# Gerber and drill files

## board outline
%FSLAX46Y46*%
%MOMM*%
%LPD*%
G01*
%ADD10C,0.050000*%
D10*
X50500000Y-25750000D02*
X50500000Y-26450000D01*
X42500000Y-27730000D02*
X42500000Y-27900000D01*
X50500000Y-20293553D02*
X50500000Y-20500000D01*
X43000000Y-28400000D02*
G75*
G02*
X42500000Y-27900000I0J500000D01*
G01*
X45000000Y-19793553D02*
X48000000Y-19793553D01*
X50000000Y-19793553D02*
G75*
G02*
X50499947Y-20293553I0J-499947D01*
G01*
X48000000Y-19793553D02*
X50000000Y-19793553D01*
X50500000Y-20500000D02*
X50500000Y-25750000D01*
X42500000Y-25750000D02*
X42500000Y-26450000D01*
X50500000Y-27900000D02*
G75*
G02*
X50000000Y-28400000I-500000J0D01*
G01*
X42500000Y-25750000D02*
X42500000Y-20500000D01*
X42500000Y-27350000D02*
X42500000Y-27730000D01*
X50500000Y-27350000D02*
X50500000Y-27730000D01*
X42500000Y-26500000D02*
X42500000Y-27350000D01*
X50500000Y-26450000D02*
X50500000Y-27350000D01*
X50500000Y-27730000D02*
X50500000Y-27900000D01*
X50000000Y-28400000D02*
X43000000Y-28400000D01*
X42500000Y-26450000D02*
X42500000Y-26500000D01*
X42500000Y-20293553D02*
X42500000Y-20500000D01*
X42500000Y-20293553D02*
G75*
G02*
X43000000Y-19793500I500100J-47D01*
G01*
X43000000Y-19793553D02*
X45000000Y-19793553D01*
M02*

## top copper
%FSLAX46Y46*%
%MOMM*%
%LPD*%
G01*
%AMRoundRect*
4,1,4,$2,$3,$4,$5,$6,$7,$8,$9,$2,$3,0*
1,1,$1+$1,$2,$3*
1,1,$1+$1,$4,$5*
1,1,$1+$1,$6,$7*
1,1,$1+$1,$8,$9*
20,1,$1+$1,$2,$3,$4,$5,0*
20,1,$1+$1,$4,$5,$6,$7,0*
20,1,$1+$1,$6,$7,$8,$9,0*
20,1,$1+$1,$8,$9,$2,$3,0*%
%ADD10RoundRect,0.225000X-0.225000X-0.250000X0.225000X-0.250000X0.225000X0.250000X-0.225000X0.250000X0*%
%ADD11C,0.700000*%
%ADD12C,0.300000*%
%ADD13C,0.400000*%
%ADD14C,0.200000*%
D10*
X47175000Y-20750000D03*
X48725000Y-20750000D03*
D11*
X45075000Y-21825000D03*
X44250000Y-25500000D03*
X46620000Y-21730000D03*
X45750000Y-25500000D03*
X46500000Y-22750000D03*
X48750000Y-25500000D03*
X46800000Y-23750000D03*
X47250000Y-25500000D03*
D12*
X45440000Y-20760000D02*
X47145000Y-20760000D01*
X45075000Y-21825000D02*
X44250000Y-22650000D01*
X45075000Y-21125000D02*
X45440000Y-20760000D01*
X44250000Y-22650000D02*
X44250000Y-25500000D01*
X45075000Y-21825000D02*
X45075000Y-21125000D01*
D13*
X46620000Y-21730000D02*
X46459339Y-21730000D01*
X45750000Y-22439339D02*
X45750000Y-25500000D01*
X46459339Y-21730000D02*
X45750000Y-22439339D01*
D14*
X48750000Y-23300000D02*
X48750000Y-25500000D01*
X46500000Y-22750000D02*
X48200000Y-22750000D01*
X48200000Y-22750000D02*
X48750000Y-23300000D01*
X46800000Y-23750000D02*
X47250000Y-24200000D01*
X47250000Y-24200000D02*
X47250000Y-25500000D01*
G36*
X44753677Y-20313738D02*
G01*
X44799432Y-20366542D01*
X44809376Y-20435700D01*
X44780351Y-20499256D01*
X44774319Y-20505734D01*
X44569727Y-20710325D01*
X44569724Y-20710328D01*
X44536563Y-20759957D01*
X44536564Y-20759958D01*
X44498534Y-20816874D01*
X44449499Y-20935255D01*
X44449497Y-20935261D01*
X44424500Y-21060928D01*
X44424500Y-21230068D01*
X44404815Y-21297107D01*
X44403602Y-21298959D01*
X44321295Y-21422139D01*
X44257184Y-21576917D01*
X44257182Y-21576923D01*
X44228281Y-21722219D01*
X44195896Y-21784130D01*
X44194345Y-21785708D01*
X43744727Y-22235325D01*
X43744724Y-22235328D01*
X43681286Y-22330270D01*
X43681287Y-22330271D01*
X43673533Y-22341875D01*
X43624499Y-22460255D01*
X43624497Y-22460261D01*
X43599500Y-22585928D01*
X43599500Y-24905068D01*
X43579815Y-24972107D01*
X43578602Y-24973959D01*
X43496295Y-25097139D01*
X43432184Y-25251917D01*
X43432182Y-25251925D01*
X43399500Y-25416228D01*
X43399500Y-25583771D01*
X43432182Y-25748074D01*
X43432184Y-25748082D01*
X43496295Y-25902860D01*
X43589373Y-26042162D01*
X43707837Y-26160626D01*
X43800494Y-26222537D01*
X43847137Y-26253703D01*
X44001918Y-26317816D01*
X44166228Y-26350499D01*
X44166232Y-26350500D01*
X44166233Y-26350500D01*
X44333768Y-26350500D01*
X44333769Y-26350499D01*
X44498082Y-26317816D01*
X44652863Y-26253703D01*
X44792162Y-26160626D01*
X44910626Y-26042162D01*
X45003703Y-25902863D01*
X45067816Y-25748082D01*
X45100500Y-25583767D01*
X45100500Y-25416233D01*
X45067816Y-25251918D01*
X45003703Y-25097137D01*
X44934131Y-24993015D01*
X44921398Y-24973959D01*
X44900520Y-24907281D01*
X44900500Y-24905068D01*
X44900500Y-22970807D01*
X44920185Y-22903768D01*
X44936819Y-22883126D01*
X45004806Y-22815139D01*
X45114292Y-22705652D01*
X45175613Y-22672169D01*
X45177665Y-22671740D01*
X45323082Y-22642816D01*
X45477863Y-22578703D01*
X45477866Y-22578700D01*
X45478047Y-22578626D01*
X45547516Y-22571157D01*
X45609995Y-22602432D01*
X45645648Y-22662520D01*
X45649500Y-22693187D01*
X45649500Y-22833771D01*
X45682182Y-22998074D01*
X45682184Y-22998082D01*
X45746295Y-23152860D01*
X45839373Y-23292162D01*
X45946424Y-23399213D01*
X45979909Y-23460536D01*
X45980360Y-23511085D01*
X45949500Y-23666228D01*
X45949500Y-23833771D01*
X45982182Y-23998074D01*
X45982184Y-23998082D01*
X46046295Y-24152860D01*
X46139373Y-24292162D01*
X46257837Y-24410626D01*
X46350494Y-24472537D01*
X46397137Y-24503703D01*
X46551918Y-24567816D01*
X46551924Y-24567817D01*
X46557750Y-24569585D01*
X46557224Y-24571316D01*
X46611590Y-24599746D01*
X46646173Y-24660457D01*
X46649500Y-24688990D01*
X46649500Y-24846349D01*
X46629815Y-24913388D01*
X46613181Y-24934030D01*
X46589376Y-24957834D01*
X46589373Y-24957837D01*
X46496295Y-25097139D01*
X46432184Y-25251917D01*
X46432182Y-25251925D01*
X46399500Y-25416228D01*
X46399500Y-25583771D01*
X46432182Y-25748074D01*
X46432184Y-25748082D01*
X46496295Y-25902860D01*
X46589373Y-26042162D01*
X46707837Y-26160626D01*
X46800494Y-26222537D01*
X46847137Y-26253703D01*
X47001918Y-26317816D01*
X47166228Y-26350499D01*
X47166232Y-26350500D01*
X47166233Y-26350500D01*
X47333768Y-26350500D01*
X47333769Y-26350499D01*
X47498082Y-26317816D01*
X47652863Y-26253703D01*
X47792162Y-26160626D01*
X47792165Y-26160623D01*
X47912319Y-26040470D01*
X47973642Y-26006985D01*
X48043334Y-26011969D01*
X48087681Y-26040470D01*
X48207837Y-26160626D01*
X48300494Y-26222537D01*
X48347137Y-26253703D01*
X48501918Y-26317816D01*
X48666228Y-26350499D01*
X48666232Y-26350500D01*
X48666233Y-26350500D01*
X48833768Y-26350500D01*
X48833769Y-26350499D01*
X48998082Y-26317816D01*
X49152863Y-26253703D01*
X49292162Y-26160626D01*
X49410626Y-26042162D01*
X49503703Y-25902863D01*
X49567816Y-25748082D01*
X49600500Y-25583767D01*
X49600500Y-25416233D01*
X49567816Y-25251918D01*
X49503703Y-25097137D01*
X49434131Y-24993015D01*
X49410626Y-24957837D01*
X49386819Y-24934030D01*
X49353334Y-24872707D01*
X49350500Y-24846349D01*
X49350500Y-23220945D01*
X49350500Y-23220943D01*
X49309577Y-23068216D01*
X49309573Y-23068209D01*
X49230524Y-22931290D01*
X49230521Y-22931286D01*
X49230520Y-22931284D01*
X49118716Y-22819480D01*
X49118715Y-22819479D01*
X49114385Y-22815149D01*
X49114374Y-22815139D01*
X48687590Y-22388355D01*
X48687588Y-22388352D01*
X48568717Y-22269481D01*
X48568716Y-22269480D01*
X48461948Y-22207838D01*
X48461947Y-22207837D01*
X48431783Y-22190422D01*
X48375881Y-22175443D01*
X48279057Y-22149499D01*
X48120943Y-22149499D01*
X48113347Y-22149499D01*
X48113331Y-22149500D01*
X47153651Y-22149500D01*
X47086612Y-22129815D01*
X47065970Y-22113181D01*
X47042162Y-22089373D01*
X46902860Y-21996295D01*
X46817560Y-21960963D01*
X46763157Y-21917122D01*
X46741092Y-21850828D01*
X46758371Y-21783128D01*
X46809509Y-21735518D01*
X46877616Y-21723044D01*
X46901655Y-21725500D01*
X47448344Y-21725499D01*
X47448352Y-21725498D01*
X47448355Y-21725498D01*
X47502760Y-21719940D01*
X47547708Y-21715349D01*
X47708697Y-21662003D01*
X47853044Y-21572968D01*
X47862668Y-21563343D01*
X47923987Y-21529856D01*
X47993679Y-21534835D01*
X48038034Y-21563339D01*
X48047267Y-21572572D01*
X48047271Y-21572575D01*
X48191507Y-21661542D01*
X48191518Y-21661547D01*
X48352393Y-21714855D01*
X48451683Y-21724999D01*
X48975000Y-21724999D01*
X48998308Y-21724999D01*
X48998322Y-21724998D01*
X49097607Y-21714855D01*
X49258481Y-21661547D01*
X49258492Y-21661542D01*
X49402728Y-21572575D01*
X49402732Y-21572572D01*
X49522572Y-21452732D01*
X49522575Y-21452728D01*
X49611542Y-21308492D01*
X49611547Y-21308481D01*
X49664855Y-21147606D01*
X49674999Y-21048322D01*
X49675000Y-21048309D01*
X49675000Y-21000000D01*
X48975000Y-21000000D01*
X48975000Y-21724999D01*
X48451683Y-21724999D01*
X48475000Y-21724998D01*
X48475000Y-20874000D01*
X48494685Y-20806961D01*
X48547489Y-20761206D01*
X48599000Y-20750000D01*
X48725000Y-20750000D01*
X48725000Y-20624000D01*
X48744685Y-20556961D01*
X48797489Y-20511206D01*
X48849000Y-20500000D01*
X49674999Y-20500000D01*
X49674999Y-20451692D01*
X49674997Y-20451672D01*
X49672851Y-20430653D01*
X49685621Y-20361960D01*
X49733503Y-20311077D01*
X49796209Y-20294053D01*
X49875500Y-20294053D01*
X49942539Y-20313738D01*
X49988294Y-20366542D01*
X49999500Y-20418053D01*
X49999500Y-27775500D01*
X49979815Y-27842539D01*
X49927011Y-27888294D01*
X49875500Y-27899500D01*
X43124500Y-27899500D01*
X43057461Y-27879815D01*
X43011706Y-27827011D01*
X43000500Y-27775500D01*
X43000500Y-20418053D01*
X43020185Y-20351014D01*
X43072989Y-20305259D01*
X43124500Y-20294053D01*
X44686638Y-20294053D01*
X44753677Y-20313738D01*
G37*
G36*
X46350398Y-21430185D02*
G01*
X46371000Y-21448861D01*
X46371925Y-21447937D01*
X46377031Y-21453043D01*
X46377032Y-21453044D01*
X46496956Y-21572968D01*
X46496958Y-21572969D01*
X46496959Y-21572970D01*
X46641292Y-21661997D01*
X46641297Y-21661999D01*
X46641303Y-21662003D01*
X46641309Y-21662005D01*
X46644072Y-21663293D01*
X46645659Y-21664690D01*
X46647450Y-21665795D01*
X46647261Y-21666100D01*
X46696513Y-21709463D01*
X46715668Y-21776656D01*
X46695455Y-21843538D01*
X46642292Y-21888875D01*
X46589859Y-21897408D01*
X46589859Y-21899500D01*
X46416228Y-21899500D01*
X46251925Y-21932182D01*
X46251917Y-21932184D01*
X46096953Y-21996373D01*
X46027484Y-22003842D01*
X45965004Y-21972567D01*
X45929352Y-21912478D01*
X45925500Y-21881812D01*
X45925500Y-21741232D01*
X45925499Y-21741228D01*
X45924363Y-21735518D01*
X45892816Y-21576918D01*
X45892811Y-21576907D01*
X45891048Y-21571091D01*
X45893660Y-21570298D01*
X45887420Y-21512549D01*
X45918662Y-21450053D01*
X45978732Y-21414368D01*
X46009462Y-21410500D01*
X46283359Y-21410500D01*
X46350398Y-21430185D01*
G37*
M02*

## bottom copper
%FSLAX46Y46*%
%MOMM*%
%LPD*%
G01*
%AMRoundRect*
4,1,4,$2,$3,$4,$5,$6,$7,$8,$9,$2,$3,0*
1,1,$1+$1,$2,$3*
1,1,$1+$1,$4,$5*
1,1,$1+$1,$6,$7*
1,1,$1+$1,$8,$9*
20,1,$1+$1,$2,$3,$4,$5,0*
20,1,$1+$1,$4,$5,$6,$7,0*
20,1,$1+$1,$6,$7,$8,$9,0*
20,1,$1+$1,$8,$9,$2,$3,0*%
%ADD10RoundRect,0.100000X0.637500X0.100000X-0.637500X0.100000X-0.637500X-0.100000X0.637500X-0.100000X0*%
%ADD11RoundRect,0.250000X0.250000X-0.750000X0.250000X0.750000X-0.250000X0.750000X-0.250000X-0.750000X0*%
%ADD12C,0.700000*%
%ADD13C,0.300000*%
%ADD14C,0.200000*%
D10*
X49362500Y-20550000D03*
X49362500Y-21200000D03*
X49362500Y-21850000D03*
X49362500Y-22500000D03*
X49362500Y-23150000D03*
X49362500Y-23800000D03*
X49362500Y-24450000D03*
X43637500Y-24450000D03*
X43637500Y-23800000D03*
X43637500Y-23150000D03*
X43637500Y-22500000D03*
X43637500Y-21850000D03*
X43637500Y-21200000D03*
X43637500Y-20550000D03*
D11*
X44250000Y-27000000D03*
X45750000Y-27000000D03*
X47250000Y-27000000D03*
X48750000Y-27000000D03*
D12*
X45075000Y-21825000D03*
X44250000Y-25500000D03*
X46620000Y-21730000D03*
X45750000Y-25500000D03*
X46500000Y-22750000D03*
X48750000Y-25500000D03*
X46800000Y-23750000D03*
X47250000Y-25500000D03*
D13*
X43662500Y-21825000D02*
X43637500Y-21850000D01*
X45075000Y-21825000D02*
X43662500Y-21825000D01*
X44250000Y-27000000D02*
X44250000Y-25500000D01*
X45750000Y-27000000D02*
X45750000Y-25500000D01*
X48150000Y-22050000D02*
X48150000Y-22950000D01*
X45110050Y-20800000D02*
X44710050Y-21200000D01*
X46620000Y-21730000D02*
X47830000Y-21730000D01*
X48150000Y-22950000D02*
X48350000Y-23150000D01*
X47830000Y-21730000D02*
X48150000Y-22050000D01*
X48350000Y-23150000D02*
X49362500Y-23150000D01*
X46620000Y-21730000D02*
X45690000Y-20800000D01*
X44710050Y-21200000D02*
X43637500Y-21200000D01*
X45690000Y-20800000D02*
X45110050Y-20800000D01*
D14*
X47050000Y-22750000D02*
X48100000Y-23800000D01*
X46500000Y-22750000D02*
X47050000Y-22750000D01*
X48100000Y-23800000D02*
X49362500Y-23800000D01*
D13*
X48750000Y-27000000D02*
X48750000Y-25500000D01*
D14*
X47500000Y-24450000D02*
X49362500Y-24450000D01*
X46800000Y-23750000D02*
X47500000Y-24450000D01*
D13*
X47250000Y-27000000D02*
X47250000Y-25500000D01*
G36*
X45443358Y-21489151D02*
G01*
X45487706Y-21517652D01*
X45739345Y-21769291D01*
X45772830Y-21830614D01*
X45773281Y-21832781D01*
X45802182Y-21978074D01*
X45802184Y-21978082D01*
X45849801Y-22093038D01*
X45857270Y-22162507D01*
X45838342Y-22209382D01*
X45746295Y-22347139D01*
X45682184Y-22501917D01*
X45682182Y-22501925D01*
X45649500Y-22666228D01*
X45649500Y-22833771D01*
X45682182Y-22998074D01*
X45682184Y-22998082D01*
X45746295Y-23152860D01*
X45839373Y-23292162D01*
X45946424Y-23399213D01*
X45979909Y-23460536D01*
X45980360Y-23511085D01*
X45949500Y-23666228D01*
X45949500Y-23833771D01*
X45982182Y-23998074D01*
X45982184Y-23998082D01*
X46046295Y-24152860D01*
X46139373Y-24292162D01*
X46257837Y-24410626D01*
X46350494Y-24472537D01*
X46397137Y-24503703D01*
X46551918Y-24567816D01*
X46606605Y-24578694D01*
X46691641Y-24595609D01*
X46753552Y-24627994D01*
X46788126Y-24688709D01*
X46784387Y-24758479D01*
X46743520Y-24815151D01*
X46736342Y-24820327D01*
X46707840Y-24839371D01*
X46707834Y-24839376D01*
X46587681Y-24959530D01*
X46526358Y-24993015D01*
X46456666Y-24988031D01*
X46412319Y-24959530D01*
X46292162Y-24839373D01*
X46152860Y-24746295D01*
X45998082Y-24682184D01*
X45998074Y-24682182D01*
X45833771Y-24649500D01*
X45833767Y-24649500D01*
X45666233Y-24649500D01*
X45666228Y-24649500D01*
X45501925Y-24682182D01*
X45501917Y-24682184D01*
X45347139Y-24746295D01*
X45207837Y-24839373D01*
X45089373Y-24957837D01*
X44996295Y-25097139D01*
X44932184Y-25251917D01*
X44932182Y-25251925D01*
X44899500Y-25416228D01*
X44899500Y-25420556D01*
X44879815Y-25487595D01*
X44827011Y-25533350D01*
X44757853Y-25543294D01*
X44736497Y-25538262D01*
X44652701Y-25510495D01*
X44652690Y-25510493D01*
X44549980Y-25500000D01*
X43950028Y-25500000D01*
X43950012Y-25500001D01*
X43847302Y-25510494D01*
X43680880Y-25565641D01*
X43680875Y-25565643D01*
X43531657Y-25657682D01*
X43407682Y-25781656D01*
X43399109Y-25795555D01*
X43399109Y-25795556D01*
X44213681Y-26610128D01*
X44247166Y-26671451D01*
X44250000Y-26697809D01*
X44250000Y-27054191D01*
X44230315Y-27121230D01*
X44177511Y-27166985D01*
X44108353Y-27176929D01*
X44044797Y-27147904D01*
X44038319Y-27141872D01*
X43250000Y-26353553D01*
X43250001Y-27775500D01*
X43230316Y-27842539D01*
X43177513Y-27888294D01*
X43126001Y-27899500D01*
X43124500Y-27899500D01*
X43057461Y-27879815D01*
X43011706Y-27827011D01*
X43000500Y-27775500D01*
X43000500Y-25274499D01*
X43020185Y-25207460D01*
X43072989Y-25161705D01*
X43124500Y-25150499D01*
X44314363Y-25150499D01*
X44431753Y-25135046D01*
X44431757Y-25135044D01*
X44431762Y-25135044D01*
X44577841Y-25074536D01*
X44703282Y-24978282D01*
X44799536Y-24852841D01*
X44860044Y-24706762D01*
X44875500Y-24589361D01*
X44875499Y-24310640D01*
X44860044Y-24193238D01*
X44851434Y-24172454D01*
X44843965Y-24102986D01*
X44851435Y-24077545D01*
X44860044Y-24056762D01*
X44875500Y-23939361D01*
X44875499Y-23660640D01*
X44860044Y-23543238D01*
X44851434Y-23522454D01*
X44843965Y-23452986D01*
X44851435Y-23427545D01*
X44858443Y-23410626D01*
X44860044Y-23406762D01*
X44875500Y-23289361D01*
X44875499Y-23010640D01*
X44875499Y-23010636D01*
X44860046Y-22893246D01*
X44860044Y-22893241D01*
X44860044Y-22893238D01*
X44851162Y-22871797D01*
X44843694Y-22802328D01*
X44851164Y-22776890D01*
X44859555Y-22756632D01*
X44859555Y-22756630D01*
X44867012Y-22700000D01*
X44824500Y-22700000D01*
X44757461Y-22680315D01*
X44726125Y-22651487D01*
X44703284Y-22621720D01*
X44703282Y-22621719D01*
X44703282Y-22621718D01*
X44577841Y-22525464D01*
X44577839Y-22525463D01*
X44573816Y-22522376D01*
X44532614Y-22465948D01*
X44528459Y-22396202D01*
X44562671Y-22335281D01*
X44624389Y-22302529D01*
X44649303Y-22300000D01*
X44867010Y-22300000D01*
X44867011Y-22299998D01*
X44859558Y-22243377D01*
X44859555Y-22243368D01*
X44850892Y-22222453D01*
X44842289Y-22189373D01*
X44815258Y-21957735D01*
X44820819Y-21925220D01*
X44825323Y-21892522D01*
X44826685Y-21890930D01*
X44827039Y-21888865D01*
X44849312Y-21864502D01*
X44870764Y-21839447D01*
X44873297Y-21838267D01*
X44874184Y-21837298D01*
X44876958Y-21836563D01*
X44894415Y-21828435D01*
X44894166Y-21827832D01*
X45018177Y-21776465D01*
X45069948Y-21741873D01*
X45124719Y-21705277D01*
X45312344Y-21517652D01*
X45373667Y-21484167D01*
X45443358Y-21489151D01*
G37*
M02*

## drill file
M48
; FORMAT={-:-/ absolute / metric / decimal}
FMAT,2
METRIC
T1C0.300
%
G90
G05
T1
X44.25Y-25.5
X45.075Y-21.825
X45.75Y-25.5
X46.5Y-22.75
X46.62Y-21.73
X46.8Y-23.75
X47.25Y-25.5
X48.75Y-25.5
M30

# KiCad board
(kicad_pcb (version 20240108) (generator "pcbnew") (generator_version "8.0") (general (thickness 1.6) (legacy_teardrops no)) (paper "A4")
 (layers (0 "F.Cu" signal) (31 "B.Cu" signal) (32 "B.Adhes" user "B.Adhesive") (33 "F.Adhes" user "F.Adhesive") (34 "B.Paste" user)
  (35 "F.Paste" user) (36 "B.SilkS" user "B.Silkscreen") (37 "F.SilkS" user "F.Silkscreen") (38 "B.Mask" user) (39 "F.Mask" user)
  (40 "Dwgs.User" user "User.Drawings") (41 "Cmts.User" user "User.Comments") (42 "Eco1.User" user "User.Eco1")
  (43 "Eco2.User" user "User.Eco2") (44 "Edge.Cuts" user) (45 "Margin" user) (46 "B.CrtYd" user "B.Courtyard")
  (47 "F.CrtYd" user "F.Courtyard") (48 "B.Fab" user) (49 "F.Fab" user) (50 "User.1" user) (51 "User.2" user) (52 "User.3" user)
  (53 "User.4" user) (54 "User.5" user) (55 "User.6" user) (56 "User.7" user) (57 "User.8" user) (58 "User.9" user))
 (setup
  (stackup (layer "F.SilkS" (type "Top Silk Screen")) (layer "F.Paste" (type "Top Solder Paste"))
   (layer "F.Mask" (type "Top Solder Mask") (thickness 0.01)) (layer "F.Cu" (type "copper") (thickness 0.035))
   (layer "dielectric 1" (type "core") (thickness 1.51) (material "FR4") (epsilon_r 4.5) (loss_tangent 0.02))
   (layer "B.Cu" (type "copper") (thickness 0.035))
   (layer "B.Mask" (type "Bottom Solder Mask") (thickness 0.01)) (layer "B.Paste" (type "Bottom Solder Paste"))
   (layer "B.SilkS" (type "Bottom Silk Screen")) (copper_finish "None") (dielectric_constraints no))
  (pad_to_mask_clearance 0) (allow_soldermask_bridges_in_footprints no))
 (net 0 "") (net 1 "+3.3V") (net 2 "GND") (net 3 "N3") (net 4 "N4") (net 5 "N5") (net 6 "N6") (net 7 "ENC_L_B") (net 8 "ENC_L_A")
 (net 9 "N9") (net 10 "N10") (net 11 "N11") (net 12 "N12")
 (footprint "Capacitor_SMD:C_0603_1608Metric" (layer "F.Cu") (at 47.95 20.75)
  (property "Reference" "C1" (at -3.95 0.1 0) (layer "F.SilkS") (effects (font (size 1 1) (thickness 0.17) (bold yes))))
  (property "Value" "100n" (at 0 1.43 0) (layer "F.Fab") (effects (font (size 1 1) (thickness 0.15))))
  (pad "1" smd roundrect (at -0.775 0) (size 0.9 0.95) (layers "F.Cu" "F.Paste" "F.Mask") (roundrect_rratio 0.25) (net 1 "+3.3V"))
  (pad "2" smd roundrect (at 0.775 0) (size 0.9 0.95) (layers "F.Cu" "F.Paste" "F.Mask") (roundrect_rratio 0.25) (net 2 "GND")))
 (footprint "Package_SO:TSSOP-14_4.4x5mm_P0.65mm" (layer "B.Cu") (at 46.5 22.5 180)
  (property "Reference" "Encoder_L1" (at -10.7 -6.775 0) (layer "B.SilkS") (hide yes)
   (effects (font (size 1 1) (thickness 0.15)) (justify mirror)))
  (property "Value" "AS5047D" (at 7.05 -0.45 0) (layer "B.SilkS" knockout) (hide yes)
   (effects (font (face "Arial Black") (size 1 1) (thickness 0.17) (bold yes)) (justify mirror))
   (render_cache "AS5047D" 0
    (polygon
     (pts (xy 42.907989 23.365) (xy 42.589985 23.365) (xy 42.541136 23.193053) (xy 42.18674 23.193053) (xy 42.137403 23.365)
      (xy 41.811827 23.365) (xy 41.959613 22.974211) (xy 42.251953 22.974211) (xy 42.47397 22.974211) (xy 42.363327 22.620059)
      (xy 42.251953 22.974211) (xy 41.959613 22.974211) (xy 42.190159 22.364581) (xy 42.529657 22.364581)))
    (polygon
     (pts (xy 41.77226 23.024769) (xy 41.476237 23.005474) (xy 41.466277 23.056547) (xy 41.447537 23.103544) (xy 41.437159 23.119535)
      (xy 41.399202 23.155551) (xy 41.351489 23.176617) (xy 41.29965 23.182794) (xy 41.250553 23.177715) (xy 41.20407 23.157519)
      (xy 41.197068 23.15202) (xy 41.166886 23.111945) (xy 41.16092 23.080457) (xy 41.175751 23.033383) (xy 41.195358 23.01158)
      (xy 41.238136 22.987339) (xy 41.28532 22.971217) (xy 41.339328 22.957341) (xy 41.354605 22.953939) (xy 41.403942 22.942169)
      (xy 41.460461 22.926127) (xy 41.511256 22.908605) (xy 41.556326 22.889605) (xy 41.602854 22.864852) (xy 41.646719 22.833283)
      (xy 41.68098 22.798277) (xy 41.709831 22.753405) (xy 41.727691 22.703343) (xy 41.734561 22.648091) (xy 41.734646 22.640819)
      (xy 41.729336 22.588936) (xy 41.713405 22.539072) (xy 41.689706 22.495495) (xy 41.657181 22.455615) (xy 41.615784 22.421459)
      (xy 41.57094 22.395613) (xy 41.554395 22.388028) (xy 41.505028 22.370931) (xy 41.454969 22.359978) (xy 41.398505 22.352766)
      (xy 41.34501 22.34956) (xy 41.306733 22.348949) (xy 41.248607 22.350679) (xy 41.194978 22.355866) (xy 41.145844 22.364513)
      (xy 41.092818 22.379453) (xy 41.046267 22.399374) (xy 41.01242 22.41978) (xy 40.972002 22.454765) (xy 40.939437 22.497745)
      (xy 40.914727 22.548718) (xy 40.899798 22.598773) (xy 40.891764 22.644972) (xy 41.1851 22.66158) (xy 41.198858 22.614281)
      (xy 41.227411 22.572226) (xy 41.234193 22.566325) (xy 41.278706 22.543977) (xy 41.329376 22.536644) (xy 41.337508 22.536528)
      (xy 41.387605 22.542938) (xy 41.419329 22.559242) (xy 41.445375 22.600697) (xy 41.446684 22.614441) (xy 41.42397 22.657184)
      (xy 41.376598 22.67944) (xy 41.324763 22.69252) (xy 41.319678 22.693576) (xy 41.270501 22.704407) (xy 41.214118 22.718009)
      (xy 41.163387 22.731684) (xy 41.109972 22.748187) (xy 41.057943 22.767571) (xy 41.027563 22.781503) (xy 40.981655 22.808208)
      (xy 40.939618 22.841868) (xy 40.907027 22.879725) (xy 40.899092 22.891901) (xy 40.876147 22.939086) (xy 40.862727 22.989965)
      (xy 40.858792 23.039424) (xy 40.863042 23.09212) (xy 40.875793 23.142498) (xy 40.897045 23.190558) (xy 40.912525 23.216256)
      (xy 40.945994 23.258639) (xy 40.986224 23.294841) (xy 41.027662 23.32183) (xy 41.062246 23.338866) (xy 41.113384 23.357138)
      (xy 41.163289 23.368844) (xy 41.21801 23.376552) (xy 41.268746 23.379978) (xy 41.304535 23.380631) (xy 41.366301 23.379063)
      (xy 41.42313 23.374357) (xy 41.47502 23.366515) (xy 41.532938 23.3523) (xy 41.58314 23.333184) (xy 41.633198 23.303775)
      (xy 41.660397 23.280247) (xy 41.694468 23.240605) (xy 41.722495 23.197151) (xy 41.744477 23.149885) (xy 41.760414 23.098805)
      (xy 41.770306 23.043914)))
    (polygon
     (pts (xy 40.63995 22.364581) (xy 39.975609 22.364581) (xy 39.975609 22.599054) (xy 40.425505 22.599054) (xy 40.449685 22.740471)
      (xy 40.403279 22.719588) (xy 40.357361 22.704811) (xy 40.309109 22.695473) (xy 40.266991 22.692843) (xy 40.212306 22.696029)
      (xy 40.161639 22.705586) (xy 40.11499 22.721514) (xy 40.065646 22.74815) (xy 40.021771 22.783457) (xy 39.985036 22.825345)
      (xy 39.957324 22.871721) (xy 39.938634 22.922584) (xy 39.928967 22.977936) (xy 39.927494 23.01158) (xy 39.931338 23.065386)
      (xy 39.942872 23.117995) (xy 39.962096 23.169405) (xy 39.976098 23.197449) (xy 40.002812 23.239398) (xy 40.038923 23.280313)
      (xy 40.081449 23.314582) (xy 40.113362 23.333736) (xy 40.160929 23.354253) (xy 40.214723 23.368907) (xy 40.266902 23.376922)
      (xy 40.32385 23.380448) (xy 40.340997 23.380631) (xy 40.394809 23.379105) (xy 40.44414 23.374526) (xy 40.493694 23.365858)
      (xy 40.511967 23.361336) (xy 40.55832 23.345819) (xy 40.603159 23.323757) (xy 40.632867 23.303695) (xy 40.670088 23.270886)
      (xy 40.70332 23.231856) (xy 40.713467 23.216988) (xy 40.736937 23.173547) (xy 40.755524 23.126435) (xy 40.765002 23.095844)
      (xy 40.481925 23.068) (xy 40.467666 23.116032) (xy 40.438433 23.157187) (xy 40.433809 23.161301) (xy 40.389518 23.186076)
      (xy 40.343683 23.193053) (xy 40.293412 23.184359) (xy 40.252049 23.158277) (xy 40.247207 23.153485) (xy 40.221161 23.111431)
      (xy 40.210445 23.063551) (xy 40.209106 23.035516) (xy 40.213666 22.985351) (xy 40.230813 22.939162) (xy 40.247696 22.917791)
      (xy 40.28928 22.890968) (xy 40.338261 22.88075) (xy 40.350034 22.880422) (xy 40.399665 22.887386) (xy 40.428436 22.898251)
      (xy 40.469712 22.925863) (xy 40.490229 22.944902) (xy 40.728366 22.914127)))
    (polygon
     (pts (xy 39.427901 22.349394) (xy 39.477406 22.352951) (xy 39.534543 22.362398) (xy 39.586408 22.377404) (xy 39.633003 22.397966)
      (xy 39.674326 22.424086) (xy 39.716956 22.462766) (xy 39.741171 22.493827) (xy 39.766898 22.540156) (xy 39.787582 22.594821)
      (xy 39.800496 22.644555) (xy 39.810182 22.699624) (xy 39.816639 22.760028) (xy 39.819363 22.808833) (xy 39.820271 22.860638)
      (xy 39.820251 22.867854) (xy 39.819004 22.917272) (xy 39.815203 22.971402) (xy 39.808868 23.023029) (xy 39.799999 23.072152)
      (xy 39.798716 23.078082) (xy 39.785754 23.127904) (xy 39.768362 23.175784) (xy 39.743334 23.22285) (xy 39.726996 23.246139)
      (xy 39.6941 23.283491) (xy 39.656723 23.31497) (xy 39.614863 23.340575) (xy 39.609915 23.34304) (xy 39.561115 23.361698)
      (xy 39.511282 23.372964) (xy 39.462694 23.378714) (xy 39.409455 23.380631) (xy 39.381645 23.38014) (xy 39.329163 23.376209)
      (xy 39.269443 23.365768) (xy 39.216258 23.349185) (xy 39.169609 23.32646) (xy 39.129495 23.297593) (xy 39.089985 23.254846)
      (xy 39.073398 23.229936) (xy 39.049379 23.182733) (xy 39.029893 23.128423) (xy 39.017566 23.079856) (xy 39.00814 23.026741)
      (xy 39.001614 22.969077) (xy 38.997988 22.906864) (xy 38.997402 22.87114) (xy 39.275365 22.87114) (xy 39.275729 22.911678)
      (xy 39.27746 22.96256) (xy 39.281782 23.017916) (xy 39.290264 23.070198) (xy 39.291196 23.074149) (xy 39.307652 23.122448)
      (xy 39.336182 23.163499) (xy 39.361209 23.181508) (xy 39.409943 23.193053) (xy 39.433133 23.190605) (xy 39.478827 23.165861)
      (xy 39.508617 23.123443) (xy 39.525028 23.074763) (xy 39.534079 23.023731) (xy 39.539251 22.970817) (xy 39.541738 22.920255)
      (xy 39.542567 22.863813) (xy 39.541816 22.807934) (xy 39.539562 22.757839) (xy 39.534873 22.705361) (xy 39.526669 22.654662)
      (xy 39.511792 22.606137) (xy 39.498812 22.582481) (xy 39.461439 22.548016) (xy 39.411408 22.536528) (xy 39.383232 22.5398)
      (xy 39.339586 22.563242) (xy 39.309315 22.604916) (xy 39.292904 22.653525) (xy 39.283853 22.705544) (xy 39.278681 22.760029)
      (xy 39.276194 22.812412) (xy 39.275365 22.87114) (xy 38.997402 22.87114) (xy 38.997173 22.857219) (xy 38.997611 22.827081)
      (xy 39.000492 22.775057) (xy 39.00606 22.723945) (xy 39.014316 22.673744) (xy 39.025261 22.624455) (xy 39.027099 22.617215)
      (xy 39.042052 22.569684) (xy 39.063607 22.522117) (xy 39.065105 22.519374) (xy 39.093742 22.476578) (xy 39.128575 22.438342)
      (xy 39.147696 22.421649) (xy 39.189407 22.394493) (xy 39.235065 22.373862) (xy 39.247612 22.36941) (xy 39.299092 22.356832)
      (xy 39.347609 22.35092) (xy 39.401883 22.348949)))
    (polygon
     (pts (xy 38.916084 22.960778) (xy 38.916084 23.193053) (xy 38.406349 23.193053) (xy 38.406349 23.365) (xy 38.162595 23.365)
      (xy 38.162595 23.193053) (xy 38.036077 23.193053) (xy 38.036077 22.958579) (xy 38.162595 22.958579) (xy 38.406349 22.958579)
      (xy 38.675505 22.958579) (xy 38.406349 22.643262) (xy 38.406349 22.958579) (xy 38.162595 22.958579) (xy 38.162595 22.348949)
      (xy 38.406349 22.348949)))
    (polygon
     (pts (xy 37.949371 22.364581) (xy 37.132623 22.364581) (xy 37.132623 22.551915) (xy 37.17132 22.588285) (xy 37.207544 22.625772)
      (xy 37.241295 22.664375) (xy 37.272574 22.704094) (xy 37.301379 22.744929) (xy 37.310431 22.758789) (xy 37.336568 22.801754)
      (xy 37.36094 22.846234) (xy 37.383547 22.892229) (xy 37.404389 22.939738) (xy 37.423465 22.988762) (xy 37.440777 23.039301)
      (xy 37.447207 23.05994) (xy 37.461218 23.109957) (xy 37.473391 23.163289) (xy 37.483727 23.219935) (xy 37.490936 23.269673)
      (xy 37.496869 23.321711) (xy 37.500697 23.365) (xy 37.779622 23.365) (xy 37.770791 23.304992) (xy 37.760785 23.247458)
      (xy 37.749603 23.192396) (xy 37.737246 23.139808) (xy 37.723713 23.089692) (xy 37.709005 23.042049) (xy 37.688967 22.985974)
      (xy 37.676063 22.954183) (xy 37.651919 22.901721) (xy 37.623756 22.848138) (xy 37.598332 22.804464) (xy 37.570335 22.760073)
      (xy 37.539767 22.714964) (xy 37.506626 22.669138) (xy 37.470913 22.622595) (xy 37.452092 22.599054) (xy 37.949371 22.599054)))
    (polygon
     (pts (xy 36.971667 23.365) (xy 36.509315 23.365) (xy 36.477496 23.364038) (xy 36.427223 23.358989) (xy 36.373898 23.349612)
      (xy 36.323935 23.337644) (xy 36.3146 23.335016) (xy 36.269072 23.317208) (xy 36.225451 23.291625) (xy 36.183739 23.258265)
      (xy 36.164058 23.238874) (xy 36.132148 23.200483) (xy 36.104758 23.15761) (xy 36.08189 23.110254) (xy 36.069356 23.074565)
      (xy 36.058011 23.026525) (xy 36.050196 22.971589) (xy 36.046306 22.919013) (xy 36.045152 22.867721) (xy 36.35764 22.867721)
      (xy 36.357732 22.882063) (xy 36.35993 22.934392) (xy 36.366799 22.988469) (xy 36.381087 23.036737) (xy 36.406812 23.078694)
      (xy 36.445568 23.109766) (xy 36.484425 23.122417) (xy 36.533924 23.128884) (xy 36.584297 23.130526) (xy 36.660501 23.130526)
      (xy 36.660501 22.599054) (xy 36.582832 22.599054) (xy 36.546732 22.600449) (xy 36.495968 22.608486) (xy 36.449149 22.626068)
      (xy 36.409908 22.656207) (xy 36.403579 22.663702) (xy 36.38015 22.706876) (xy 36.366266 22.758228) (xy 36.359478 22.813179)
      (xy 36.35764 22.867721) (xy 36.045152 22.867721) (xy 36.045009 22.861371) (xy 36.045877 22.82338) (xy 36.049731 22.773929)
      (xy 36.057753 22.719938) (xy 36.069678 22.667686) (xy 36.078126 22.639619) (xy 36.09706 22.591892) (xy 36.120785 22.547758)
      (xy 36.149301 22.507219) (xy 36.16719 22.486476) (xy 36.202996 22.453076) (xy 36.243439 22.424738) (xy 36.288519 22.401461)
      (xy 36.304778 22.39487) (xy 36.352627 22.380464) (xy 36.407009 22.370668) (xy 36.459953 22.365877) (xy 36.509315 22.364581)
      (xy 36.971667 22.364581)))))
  (pad "1" smd roundrect (at -2.8625 1.95 180) (size 1.475 0.4) (layers "B.Cu" "B.Paste" "B.Mask") (roundrect_rratio 0.25) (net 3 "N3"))
  (pad "2" smd roundrect (at -2.8625 1.3 180) (size 1.475 0.4) (layers "B.Cu" "B.Paste" "B.Mask") (roundrect_rratio 0.25) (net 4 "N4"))
  (pad "3" smd roundrect (at -2.8625 0.65 180) (size 1.475 0.4) (layers "B.Cu" "B.Paste" "B.Mask") (roundrect_rratio 0.25) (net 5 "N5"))
  (pad "4" smd roundrect (at -2.8625 0 180) (size 1.475 0.4) (layers "B.Cu" "B.Paste" "B.Mask") (roundrect_rratio 0.25) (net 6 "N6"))
  (pad "5" smd roundrect (at -2.8625 -0.65 180) (size 1.475 0.4) (layers "B.Cu" "B.Paste" "B.Mask") (roundrect_rratio 0.25) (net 2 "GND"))
  (pad "6" smd roundrect (at -2.8625 -1.3 180) (size 1.475 0.4) (layers "B.Cu" "B.Paste" "B.Mask") (roundrect_rratio 0.25) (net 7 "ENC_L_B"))
  (pad "7" smd roundrect (at -2.8625 -1.95 180) (size 1.475 0.4) (layers "B.Cu" "B.Paste" "B.Mask") (roundrect_rratio 0.25)
   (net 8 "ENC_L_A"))
  (pad "8" smd roundrect (at 2.8625 -1.95 180) (size 1.475 0.4) (layers "B.Cu" "B.Paste" "B.Mask") (roundrect_rratio 0.25) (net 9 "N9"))
  (pad "9" smd roundrect (at 2.8625 -1.3 180) (size 1.475 0.4) (layers "B.Cu" "B.Paste" "B.Mask") (roundrect_rratio 0.25) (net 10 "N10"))
  (pad "10" smd roundrect (at 2.8625 -0.65 180) (size 1.475 0.4) (layers "B.Cu" "B.Paste" "B.Mask") (roundrect_rratio 0.25) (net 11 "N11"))
  (pad "11" smd roundrect (at 2.8625 0 180) (size 1.475 0.4) (layers "B.Cu" "B.Paste" "B.Mask") (roundrect_rratio 0.25) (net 1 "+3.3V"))
  (pad "12" smd roundrect (at 2.8625 0.65 180) (size 1.475 0.4) (layers "B.Cu" "B.Paste" "B.Mask") (roundrect_rratio 0.25) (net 1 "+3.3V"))
  (pad "13" smd roundrect (at 2.8625 1.3 180) (size 1.475 0.4) (layers "B.Cu" "B.Paste" "B.Mask") (roundrect_rratio 0.25) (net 2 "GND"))
  (pad "14" smd roundrect (at 2.8625 1.95 180) (size 1.475 0.4) (layers "B.Cu" "B.Paste" "B.Mask") (roundrect_rratio 0.25) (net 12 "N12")))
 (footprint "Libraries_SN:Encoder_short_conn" (layer "B.Cu") (at 46.25 28 180)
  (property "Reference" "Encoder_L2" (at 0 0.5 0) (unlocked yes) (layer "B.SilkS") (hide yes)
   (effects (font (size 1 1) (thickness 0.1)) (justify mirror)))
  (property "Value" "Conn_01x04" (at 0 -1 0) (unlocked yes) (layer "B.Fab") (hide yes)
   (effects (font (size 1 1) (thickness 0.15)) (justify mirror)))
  (pad "1" smd roundrect (at 2 1 90) (size 2 1) (layers "B.Cu" "B.Paste" "B.Mask") (roundrect_rratio 0.25) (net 1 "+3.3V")
   (thermal_bridge_angle 45))
  (pad "2" smd roundrect (at 0.5 1 90) (size 2 1) (layers "B.Cu" "B.Paste" "B.Mask") (roundrect_rratio 0.25) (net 2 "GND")
   (thermal_bridge_angle 45))
  (pad "3" smd roundrect (at -1 1 90) (size 2 1) (layers "B.Cu" "B.Paste" "B.Mask") (roundrect_rratio 0.25) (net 8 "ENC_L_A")
   (thermal_bridge_angle 45))
  (pad "4" smd roundrect (at -2.5 1 90) (size 2 1) (layers "B.Cu" "B.Paste" "B.Mask") (roundrect_rratio 0.25) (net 7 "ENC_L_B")
   (thermal_bridge_angle 45)))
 (gr_line (start 50.5 25.75) (end 50.5 26.45) (stroke (width 0.05) (type default)) (layer "Edge.Cuts"))
 (gr_line (start 42.5 27.73) (end 42.5 27.9) (stroke (width 0.05) (type default)) (layer "Edge.Cuts"))
 (gr_line (start 50.5 20.293553) (end 50.5 20.5) (stroke (width 0.05) (type default)) (layer "Edge.Cuts"))
 (gr_arc (start 43 28.4) (mid 42.646447 28.253553) (end 42.5 27.9) (stroke (width 0.05) (type default)) (layer "Edge.Cuts"))
 (gr_line (start 45 19.793553) (end 48 19.793553) (stroke (width 0.05) (type default)) (layer "Edge.Cuts"))
 (gr_arc (start 50 19.793553) (mid 50.35357 19.939997) (end 50.5 20.293553) (stroke (width 0.05) (type default)) (layer "Edge.Cuts"))
 (gr_line (start 48 19.793553) (end 50 19.793553) (stroke (width 0.05) (type default)) (layer "Edge.Cuts"))
 (gr_line (start 50.5 20.5) (end 50.5 25.75) (stroke (width 0.05) (type default)) (layer "Edge.Cuts"))
 (gr_line (start 42.5 25.75) (end 42.5 26.45) (stroke (width 0.05) (type default)) (layer "Edge.Cuts"))
 (gr_arc (start 50.5 27.9) (mid 50.353553 28.253553) (end 50 28.4) (stroke (width 0.05) (type default)) (layer "Edge.Cuts"))
 (gr_line (start 42.5 25.75) (end 42.5 20.5) (stroke (width 0.05) (type default)) (layer "Edge.Cuts"))
 (gr_line (start 42.5 27.35) (end 42.5 27.73) (stroke (width 0.05) (type default)) (layer "Edge.Cuts"))
 (gr_line (start 50.5 27.35) (end 50.5 27.73) (stroke (width 0.05) (type default)) (layer "Edge.Cuts"))
 (gr_line (start 42.5 26.5) (end 42.5 27.35) (stroke (width 0.05) (type default)) (layer "Edge.Cuts"))
 (gr_line (start 50.5 26.45) (end 50.5 27.35) (stroke (width 0.05) (type default)) (layer "Edge.Cuts"))
 (gr_line (start 50.5 27.73) (end 50.5 27.9) (stroke (width 0.05) (type default)) (layer "Edge.Cuts"))
 (gr_line (start 50 28.4) (end 43 28.4) (stroke (width 0.05) (type default)) (layer "Edge.Cuts"))
 (gr_line (start 42.5 26.45) (end 42.5 26.5) (stroke (width 0.05) (type default)) (layer "Edge.Cuts"))
 (gr_line (start 42.5 20.293553) (end 42.5 20.5) (stroke (width 0.05) (type default)) (layer "Edge.Cuts"))
 (gr_arc (start 42.5 20.293553) (mid 42.646463 19.94003) (end 43 19.793553) (stroke (width 0.05) (type default)) (layer "Edge.Cuts"))
 (gr_line (start 43 19.793553) (end 45 19.793553) (stroke (width 0.05) (type default)) (layer "Edge.Cuts"))
 (segment (start 45.44 20.76) (end 47.145 20.76) (width 0.3) (layer "F.Cu") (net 1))
 (segment (start 45.075 21.825) (end 44.25 22.65) (width 0.3) (layer "F.Cu") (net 1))
 (segment (start 45.075 21.125) (end 45.44 20.76) (width 0.3) (layer "F.Cu") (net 1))
 (segment (start 44.25 22.65) (end 44.25 25.5) (width 0.3) (layer "F.Cu") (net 1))
 (segment (start 45.075 21.825) (end 45.075 21.125) (width 0.3) (layer "F.Cu") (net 1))
 (via (at 45.075 21.825) (size 0.7) (drill 0.3) (layers "F.Cu" "B.Cu") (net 1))
 (via (at 44.25 25.5) (size 0.7) (drill 0.3) (layers "F.Cu" "B.Cu") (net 1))
 (segment (start 43.6625 21.825) (end 43.6375 21.85) (width 0.3) (layer "B.Cu") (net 1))
 (segment (start 45.075 21.825) (end 43.6625 21.825) (width 0.3) (layer "B.Cu") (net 1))
 (segment (start 44.25 27) (end 44.25 25.5) (width 0.3) (layer "B.Cu") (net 1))
 (segment (start 46.62 21.73) (end 46.459339 21.73) (width 0.4) (layer "F.Cu") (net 2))
 (segment (start 45.75 22.439339) (end 45.75 25.5) (width 0.4) (layer "F.Cu") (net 2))
 (segment (start 46.459339 21.73) (end 45.75 22.439339) (width 0.4) (layer "F.Cu") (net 2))
 (via (at 46.62 21.73) (size 0.7) (drill 0.3) (layers "F.Cu" "B.Cu") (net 2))
 (via (at 45.75 25.5) (size 0.7) (drill 0.3) (layers "F.Cu" "B.Cu") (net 2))
 (segment (start 45.75 27) (end 45.75 25.5) (width 0.3) (layer "B.Cu") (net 2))
 (segment (start 48.15 22.05) (end 48.15 22.95) (width 0.3) (layer "B.Cu") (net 2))
 (segment (start 45.11005 20.8) (end 44.71005 21.2) (width 0.3) (layer "B.Cu") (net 2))
 (segment (start 46.62 21.73) (end 47.83 21.73) (width 0.3) (layer "B.Cu") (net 2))
 (segment (start 48.15 22.95) (end 48.35 23.15) (width 0.3) (layer "B.Cu") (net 2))
 (segment (start 47.83 21.73) (end 48.15 22.05) (width 0.3) (layer "B.Cu") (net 2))
 (segment (start 48.35 23.15) (end 49.3625 23.15) (width 0.3) (layer "B.Cu") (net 2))
 (segment (start 46.62 21.73) (end 45.69 20.8) (width 0.3) (layer "B.Cu") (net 2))
 (segment (start 44.71005 21.2) (end 43.6375 21.2) (width 0.3) (layer "B.Cu") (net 2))
 (segment (start 45.69 20.8) (end 45.11005 20.8) (width 0.3) (layer "B.Cu") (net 2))
 (segment (start 48.75 23.3) (end 48.75 25.5) (width 0.2) (layer "F.Cu") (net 7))
 (segment (start 46.5 22.75) (end 48.2 22.75) (width 0.2) (layer "F.Cu") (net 7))
 (segment (start 48.2 22.75) (end 48.75 23.3) (width 0.2) (layer "F.Cu") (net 7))
 (via (at 46.5 22.75) (size 0.7) (drill 0.3) (layers "F.Cu" "B.Cu") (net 7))
 (via (at 48.75 25.5) (size 0.7) (drill 0.3) (layers "F.Cu" "B.Cu") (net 7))
 (segment (start 47.05 22.75) (end 48.1 23.8) (width 0.2) (layer "B.Cu") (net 7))
 (segment (start 46.5 22.75) (end 47.05 22.75) (width 0.2) (layer "B.Cu") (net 7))
 (segment (start 48.1 23.8) (end 49.3625 23.8) (width 0.2) (layer "B.Cu") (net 7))
 (segment (start 48.75 27) (end 48.75 25.5) (width 0.3) (layer "B.Cu") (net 7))
 (segment (start 46.8 23.75) (end 47.25 24.2) (width 0.2) (layer "F.Cu") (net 8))
 (segment (start 47.25 24.2) (end 47.25 25.5) (width 0.2) (layer "F.Cu") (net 8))
 (via (at 46.8 23.75) (size 0.7) (drill 0.3) (layers "F.Cu" "B.Cu") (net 8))
 (via (at 47.25 25.5) (size 0.7) (drill 0.3) (layers "F.Cu" "B.Cu") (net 8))
 (segment (start 47.5 24.45) (end 49.3625 24.45) (width 0.2) (layer "B.Cu") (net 8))
 (segment (start 46.8 23.75) (end 47.5 24.45) (width 0.2) (layer "B.Cu") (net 8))
 (segment (start 47.25 27) (end 47.25 25.5) (width 0.3) (layer "B.Cu") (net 8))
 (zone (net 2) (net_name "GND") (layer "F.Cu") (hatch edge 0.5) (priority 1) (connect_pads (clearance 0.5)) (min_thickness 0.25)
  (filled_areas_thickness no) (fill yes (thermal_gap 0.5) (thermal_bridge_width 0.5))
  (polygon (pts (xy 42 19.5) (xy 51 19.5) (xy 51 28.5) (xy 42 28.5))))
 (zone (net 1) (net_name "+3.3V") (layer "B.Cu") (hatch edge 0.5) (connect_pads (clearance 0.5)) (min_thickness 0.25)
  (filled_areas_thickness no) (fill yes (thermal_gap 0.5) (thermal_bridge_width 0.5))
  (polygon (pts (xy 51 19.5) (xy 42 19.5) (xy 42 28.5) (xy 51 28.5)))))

